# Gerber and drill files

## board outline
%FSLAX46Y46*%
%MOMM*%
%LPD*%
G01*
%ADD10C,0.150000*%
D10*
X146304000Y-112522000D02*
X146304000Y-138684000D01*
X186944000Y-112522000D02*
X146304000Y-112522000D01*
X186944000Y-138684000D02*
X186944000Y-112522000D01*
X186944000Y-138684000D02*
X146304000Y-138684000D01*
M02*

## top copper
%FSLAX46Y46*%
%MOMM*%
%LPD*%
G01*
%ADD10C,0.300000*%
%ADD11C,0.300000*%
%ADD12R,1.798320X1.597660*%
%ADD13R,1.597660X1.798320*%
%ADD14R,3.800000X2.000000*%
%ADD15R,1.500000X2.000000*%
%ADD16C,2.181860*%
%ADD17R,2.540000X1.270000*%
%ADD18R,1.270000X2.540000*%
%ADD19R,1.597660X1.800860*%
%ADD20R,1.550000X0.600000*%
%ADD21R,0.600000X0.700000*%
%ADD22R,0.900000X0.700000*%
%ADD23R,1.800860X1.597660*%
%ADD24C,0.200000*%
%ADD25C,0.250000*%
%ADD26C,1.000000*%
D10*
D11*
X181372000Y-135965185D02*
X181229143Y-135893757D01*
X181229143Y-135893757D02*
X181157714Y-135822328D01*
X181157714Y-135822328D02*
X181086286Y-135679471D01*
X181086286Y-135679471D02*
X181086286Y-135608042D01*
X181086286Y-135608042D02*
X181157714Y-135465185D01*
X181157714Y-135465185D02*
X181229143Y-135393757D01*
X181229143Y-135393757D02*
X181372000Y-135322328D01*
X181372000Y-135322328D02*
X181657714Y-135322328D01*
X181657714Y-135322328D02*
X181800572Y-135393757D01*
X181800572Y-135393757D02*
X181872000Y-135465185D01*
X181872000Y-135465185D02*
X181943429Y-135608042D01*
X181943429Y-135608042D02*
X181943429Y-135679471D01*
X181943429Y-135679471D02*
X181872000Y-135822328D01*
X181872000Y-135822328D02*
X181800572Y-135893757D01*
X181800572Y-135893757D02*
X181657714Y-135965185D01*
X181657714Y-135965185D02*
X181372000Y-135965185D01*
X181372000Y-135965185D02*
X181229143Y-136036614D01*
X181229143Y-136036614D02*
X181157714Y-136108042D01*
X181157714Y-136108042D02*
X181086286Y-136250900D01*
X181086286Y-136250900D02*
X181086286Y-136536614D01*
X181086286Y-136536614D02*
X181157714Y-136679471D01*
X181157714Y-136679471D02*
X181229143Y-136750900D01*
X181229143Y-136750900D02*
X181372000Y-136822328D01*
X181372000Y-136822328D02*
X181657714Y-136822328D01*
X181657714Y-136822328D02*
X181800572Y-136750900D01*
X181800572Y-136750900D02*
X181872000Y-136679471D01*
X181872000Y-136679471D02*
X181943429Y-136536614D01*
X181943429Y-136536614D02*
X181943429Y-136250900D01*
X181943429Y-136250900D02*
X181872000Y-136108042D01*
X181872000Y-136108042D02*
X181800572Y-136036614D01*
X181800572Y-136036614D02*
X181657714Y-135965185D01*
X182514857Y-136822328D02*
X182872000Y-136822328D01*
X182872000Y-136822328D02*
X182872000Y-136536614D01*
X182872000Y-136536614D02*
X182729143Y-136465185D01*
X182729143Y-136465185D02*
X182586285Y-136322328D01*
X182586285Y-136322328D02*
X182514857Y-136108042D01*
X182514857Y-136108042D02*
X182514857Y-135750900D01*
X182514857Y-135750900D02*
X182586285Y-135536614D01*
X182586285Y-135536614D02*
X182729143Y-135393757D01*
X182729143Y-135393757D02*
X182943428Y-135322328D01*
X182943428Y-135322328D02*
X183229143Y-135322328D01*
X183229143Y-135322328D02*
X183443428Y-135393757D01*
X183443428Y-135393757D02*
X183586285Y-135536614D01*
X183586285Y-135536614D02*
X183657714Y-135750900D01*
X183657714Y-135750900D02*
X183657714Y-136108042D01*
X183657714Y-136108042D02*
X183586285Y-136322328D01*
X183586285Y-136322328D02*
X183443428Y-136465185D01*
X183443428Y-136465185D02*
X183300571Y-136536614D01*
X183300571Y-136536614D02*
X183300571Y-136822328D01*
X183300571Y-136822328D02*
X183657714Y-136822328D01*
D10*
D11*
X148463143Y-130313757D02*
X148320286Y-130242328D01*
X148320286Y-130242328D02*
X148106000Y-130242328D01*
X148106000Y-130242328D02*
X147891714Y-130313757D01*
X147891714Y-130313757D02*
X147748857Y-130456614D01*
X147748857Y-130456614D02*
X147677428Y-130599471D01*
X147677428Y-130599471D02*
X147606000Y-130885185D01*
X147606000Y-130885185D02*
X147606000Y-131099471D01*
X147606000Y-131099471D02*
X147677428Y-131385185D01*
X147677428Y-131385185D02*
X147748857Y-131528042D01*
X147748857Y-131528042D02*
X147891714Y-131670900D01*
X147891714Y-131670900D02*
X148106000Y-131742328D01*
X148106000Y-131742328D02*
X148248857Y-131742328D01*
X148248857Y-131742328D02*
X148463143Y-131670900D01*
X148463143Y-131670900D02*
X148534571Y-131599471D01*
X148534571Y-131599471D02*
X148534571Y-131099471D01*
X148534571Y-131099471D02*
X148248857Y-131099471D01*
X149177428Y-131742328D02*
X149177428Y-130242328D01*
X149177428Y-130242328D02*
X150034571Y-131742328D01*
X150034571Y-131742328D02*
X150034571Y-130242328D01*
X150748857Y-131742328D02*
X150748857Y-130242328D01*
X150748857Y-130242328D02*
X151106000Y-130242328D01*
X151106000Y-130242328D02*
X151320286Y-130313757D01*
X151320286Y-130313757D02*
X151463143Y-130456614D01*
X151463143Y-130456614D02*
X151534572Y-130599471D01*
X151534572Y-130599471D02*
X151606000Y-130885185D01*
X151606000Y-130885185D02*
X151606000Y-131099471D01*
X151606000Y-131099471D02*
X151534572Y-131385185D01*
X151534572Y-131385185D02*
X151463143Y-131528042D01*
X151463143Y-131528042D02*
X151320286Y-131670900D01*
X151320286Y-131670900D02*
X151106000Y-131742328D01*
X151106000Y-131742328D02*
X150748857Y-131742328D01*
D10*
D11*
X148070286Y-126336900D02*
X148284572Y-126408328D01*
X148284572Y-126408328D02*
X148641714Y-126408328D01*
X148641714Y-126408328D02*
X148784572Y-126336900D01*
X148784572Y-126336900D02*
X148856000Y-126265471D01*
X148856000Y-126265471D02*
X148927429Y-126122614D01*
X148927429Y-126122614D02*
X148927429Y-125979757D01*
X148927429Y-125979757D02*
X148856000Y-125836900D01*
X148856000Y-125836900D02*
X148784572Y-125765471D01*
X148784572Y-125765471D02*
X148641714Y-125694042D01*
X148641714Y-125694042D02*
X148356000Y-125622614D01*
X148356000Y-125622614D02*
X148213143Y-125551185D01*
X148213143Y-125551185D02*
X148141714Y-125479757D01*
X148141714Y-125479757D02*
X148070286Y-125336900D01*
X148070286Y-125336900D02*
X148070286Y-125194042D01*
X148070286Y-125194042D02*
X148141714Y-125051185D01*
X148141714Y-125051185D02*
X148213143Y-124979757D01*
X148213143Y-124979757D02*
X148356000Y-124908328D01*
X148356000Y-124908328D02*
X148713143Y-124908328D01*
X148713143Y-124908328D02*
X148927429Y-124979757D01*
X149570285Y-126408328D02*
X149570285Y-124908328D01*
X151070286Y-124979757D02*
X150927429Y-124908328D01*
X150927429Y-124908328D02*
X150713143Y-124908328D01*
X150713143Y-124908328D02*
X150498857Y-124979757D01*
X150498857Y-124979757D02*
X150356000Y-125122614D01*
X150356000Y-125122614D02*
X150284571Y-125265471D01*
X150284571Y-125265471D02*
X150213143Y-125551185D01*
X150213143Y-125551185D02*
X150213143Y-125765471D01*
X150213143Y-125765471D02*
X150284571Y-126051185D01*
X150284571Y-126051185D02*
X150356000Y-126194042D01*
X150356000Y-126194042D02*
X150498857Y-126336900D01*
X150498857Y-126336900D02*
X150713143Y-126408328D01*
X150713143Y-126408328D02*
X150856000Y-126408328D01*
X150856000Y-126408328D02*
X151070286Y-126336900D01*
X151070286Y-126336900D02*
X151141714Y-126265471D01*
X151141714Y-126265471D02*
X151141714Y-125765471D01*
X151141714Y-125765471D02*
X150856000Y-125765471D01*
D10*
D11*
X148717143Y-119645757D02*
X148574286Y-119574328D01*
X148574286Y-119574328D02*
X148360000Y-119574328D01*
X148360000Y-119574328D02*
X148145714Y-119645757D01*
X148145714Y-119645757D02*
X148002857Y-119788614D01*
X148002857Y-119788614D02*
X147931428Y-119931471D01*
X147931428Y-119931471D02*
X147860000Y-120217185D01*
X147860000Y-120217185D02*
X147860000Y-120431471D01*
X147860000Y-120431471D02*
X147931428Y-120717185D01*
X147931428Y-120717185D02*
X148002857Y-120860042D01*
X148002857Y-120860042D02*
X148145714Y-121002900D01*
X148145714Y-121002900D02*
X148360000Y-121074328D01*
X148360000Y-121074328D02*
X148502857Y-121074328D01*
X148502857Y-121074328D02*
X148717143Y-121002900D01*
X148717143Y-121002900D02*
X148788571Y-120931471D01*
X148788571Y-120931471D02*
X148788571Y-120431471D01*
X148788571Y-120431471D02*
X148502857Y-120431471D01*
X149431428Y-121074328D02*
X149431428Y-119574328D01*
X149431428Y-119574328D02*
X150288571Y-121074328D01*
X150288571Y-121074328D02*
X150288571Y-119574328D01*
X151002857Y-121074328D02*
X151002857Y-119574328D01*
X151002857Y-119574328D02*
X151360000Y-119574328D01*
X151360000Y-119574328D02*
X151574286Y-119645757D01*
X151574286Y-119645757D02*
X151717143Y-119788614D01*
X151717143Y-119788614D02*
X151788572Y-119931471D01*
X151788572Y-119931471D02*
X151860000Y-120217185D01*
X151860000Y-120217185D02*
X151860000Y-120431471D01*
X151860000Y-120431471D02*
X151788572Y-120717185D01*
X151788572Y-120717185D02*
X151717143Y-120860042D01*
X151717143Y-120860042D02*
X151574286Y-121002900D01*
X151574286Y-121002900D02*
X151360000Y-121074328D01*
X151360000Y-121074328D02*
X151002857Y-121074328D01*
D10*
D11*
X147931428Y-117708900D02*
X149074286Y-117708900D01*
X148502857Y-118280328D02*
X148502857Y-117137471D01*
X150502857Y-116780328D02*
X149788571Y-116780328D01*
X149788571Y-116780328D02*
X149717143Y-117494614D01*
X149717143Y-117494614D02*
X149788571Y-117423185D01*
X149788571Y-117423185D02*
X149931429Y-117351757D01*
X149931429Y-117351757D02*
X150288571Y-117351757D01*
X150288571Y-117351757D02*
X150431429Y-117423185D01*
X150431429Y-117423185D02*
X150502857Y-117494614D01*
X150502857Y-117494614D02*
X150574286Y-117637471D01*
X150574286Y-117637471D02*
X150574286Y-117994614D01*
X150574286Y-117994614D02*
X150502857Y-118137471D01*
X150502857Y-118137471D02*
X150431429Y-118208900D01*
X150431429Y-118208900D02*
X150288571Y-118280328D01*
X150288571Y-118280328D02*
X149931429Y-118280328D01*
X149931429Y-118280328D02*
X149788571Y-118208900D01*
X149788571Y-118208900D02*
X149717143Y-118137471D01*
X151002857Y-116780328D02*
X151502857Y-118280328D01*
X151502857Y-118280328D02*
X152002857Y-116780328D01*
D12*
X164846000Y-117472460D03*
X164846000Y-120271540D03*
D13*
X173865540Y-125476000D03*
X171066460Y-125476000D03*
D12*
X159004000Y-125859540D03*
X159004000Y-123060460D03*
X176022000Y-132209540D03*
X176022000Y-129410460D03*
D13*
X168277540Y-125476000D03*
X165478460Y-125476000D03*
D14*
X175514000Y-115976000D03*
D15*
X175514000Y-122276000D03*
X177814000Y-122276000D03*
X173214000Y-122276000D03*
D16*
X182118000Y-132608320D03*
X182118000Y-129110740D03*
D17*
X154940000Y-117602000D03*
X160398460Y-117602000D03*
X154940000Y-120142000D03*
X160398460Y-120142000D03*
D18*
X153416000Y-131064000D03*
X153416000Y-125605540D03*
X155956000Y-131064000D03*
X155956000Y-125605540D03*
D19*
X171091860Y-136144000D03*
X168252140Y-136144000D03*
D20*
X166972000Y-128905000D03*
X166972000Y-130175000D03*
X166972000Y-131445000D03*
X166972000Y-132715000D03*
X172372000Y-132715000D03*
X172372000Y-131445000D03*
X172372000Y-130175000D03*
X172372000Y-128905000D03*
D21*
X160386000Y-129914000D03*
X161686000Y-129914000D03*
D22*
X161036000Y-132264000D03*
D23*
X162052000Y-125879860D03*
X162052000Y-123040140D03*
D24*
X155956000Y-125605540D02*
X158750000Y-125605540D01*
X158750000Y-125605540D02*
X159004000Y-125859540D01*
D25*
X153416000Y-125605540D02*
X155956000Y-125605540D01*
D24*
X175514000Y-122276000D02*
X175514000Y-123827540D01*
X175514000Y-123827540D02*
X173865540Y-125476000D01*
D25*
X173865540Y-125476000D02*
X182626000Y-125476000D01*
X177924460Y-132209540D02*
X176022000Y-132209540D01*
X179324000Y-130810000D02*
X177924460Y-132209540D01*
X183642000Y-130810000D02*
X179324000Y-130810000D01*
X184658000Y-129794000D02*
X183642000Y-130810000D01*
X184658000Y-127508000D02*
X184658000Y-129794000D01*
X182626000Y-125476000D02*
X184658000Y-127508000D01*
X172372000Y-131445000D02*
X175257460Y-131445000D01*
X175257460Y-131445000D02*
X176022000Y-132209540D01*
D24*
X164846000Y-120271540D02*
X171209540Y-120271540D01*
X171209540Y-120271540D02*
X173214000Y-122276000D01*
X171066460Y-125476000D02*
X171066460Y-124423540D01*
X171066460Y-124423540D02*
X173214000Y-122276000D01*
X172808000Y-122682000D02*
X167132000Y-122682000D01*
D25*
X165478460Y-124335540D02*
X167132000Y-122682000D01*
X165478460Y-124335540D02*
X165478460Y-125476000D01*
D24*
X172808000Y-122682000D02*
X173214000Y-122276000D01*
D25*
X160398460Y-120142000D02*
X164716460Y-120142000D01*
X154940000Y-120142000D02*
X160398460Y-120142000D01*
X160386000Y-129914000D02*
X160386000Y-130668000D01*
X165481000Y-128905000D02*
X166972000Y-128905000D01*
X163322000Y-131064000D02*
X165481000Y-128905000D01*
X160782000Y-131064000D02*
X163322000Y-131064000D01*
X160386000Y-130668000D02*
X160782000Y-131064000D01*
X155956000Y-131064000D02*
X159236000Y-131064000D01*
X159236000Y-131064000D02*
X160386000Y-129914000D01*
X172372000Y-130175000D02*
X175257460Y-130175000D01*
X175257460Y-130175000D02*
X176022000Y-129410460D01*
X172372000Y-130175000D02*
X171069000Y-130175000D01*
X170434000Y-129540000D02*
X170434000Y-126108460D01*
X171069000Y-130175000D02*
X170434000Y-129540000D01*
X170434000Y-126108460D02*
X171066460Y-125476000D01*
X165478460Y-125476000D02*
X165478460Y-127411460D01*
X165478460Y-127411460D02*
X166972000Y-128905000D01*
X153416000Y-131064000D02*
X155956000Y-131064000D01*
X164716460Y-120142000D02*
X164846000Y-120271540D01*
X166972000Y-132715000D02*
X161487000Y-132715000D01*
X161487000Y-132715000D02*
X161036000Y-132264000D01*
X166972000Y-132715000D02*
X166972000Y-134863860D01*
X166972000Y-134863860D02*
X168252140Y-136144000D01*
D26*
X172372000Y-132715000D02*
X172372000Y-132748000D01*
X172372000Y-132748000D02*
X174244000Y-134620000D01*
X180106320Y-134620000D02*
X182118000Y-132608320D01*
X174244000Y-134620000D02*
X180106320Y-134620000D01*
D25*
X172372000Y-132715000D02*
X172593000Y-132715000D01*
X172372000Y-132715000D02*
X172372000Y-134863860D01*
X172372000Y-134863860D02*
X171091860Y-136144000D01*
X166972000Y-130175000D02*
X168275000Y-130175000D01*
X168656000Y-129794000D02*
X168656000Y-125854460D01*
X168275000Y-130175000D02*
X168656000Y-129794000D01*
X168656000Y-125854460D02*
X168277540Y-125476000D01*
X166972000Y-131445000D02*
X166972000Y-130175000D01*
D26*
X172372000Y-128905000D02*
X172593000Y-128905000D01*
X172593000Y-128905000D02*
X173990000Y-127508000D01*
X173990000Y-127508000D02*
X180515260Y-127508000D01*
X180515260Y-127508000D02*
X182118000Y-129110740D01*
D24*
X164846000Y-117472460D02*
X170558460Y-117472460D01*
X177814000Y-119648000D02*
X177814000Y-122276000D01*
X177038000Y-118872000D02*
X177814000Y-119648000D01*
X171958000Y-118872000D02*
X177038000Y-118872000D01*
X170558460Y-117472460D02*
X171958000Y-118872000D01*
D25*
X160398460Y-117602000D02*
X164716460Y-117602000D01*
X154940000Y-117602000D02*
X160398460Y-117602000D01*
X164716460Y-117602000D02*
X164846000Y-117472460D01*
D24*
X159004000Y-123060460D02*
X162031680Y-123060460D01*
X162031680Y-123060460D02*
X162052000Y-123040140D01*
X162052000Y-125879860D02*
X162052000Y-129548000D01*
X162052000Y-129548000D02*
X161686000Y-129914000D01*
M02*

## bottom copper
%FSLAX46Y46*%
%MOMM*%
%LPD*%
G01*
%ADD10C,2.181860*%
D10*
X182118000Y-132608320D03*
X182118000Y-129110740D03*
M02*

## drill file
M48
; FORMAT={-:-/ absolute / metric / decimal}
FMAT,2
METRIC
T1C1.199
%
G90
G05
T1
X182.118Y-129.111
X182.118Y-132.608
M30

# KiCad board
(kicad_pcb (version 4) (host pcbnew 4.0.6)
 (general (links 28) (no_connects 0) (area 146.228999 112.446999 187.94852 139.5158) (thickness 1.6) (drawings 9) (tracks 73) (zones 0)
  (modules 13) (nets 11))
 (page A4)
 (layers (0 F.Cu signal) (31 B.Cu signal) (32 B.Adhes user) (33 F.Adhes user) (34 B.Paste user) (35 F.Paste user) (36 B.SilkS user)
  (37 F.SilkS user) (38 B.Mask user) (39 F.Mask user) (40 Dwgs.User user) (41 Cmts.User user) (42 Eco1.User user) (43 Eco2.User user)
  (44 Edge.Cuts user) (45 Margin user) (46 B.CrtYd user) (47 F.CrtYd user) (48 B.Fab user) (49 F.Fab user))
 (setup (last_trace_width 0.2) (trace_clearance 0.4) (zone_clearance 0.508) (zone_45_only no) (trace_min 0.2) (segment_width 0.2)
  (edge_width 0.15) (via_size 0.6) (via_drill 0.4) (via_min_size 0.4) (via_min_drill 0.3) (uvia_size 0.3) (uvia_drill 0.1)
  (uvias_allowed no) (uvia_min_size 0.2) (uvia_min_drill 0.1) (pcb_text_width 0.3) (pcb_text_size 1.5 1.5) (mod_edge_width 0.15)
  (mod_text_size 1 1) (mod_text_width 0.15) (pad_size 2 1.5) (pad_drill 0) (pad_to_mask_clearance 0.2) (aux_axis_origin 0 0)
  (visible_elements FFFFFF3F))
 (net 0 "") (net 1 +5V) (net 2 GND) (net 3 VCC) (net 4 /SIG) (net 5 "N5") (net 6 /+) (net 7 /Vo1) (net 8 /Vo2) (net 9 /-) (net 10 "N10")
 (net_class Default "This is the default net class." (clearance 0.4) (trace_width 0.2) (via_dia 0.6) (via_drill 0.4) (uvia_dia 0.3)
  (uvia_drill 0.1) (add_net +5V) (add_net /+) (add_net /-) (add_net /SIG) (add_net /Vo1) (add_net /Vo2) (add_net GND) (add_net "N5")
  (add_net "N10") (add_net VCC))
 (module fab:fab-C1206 (layer F.Cu) (at 164.846 118.872 270)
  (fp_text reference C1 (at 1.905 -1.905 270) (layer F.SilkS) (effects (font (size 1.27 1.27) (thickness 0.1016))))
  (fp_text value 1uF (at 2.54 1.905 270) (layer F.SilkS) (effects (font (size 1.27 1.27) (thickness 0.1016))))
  (pad 1 smd rect (at -1.39954 0 270) (size 1.59766 1.79832) (layers F.Cu F.Paste F.Mask) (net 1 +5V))
  (pad 2 smd rect (at 1.39954 0 270) (size 1.59766 1.79832) (layers F.Cu F.Paste F.Mask) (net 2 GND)))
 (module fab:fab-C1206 (layer F.Cu) (at 172.466 125.476 180)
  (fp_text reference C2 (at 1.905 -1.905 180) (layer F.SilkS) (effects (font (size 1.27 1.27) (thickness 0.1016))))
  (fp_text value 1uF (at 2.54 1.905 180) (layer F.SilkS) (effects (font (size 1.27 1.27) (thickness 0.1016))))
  (pad 1 smd rect (at -1.39954 0 180) (size 1.59766 1.79832) (layers F.Cu F.Paste F.Mask) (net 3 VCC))
  (pad 2 smd rect (at 1.39954 0 180) (size 1.59766 1.79832) (layers F.Cu F.Paste F.Mask) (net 2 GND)))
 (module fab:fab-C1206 (layer F.Cu) (at 159.004 124.46 90)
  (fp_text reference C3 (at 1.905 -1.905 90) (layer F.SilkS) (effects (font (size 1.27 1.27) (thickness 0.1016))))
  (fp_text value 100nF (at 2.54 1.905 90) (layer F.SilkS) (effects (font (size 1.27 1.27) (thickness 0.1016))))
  (pad 1 smd rect (at -1.39954 0 90) (size 1.59766 1.79832) (layers F.Cu F.Paste F.Mask) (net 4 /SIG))
  (pad 2 smd rect (at 1.39954 0 90) (size 1.59766 1.79832) (layers F.Cu F.Paste F.Mask) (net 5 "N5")))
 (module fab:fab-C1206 (layer F.Cu) (at 176.022 130.81 90)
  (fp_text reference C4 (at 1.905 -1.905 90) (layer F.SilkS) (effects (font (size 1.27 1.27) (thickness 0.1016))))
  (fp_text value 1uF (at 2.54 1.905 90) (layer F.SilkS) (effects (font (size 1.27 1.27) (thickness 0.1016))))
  (pad 1 smd rect (at -1.39954 0 90) (size 1.59766 1.79832) (layers F.Cu F.Paste F.Mask) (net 3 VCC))
  (pad 2 smd rect (at 1.39954 0 90) (size 1.59766 1.79832) (layers F.Cu F.Paste F.Mask) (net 2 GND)))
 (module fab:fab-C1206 (layer F.Cu) (at 166.878 125.476 180)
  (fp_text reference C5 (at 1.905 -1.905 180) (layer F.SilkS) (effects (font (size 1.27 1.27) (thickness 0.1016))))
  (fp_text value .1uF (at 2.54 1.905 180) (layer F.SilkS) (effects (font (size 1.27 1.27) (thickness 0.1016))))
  (pad 1 smd rect (at -1.39954 0 180) (size 1.59766 1.79832) (layers F.Cu F.Paste F.Mask) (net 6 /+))
  (pad 2 smd rect (at 1.39954 0 180) (size 1.59766 1.79832) (layers F.Cu F.Paste F.Mask) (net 2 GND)))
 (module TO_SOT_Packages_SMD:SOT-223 (layer F.Cu) (at 175.514 119.126 90)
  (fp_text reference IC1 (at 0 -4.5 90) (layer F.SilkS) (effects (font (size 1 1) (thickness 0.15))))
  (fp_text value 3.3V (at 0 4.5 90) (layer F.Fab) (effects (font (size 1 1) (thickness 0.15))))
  (pad 4 smd rect (at 3.15 0 90) (size 2 3.8) (layers F.Cu F.Paste F.Mask))
  (pad 1 smd rect (at -3.15 0 90) (size 2 1.5) (layers F.Cu F.Paste F.Mask) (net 3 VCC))
  (pad 2 smd rect (at -3.15 2.3 90) (size 2 1.5) (layers F.Cu F.Paste F.Mask) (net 1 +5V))
  (pad 3 smd rect (at -3.15 -2.3 90) (size 2 1.5) (layers F.Cu F.Paste F.Mask) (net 2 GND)))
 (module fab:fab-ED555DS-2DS (layer F.Cu) (at 182.118 130.81 270)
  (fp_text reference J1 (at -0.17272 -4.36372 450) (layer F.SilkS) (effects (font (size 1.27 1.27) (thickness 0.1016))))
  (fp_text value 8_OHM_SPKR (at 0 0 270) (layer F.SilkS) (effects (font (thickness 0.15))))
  (pad 1 thru_hole circle (at 1.79832 0 270) (size 2.18186 2.18186) (drill 1.19888) (layers *.Cu F.Paste F.SilkS F.Mask) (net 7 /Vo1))
  (pad 2 thru_hole circle (at -1.69926 0 270) (size 2.18186 2.18186) (drill 1.19888) (layers *.Cu F.Paste F.SilkS F.Mask) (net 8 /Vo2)))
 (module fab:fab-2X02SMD (layer F.Cu) (at 157.48 118.872)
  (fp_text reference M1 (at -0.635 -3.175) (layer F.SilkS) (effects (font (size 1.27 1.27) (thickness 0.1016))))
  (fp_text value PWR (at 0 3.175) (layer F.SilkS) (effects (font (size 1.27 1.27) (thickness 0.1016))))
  (pad 1 smd rect (at -2.54 -1.27) (size 2.54 1.27) (layers F.Cu F.Paste F.Mask) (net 1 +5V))
  (pad 2 smd rect (at 2.91846 -1.27) (size 2.54 1.27) (layers F.Cu F.Paste F.Mask) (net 1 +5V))
  (pad 3 smd rect (at -2.54 1.27) (size 2.54 1.27) (layers F.Cu F.Paste F.Mask) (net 2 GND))
  (pad 4 smd rect (at 2.91846 1.27) (size 2.54 1.27) (layers F.Cu F.Paste F.Mask) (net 2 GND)))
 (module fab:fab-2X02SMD (layer F.Cu) (at 154.686 128.524 90)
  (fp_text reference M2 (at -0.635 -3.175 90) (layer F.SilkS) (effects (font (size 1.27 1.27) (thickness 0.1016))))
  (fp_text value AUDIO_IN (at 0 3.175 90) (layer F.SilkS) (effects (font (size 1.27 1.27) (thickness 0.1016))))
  (pad 1 smd rect (at -2.54 -1.27 90) (size 2.54 1.27) (layers F.Cu F.Paste F.Mask) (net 2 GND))
  (pad 2 smd rect (at 2.91846 -1.27 90) (size 2.54 1.27) (layers F.Cu F.Paste F.Mask) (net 4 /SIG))
  (pad 3 smd rect (at -2.54 1.27 90) (size 2.54 1.27) (layers F.Cu F.Paste F.Mask) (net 2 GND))
  (pad 4 smd rect (at 2.91846 1.27 90) (size 2.54 1.27) (layers F.Cu F.Paste F.Mask) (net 4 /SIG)))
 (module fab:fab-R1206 (layer F.Cu) (at 169.672 136.144 180)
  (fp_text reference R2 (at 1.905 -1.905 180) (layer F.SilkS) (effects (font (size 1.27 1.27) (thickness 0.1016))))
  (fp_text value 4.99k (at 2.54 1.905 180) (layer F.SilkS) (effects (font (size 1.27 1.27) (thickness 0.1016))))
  (pad 1 smd rect (at -1.41986 0 180) (size 1.59766 1.80086) (layers F.Cu F.Paste F.Mask) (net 7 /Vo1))
  (pad 2 smd rect (at 1.41986 0 180) (size 1.59766 1.80086) (layers F.Cu F.Paste F.Mask) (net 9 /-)))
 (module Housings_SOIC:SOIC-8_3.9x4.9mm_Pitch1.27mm (layer F.Cu) (at 169.672 130.81)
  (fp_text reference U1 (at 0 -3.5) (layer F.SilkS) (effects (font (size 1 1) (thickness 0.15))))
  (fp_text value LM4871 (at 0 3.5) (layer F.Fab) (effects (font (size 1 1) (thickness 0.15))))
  (pad 1 smd rect (at -2.7 -1.905) (size 1.55 0.6) (layers F.Cu F.Paste F.Mask) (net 2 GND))
  (pad 2 smd rect (at -2.7 -0.635) (size 1.55 0.6) (layers F.Cu F.Paste F.Mask) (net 6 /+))
  (pad 3 smd rect (at -2.7 0.635) (size 1.55 0.6) (layers F.Cu F.Paste F.Mask) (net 6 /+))
  (pad 4 smd rect (at -2.7 1.905) (size 1.55 0.6) (layers F.Cu F.Paste F.Mask) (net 9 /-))
  (pad 5 smd rect (at 2.7 1.905) (size 1.55 0.6) (layers F.Cu F.Paste F.Mask) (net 7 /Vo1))
  (pad 6 smd rect (at 2.7 0.635) (size 1.55 0.6) (layers F.Cu F.Paste F.Mask) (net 3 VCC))
  (pad 7 smd rect (at 2.7 -0.635) (size 1.55 0.6) (layers F.Cu F.Paste F.Mask) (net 2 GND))
  (pad 8 smd rect (at 2.7 -1.905) (size 1.55 0.6) (layers F.Cu F.Paste F.Mask) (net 8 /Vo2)))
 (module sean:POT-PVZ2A (layer F.Cu) (at 161.036 131.064 180)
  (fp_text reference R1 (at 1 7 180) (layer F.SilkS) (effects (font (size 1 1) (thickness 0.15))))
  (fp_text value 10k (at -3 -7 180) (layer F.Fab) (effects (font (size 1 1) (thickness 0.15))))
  (pad 3 smd rect (at 0.65 1.15 180) (size 0.6 0.7) (layers F.Cu F.Paste F.Mask) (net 2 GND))
  (pad 1 smd rect (at -0.65 1.15 180) (size 0.6 0.7) (layers F.Cu F.Paste F.Mask) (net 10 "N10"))
  (pad 2 smd rect (at 0 -1.2 180) (size 0.9 0.7) (layers F.Cu F.Paste F.Mask) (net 9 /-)))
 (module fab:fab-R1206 (layer F.Cu) (at 162.052 124.46 90)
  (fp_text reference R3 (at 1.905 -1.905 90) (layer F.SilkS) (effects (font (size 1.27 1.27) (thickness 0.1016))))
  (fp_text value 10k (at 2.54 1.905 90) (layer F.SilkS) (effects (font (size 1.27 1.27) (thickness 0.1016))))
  (pad 1 smd rect (at -1.41986 0 90) (size 1.59766 1.80086) (layers F.Cu F.Paste F.Mask) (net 10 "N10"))
  (pad 2 smd rect (at 1.41986 0 90) (size 1.59766 1.80086) (layers F.Cu F.Paste F.Mask) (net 5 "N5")))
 (gr_line (start 146.304 112.522) (end 146.304 138.684) (angle 90) (layer Edge.Cuts) (width 0.15))
 (gr_line (start 186.944 112.522) (end 146.304 112.522) (angle 90) (layer Edge.Cuts) (width 0.15))
 (gr_line (start 186.944 138.684) (end 186.944 112.522) (angle 90) (layer Edge.Cuts) (width 0.15))
 (gr_line (start 186.944 138.684) (end 146.304 138.684) (angle 90) (layer Edge.Cuts) (width 0.15))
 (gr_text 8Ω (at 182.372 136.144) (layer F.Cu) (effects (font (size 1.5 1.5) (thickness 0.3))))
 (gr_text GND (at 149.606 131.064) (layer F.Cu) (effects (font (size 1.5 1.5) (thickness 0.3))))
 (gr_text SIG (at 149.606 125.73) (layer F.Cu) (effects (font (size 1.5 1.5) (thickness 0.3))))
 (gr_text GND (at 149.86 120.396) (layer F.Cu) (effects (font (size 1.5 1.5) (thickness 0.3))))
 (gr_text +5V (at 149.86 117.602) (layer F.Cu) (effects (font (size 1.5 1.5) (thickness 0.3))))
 (segment (start 155.956 125.60554) (end 158.75 125.60554) (width 0.2) (layer F.Cu) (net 4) (status C00000))
 (segment (start 158.75 125.60554) (end 159.004 125.85954) (width 0.2) (layer F.Cu) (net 4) (status C00000))
 (segment (start 153.416 125.60554) (end 155.956 125.60554) (width 0.25) (layer F.Cu) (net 4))
 (segment (start 175.514 122.276) (end 175.514 123.82754) (width 0.2) (layer F.Cu) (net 3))
 (segment (start 175.514 123.82754) (end 173.86554 125.476) (width 0.2) (layer F.Cu) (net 3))
 (segment (start 173.86554 125.476) (end 182.626 125.476) (width 0.25) (layer F.Cu) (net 3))
 (segment (start 177.92446 132.20954) (end 176.022 132.20954) (width 0.25) (layer F.Cu) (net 3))
 (segment (start 179.324 130.81) (end 177.92446 132.20954) (width 0.25) (layer F.Cu) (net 3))
 (segment (start 183.642 130.81) (end 179.324 130.81) (width 0.25) (layer F.Cu) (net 3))
 (segment (start 184.658 129.794) (end 183.642 130.81) (width 0.25) (layer F.Cu) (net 3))
 (segment (start 184.658 127.508) (end 184.658 129.794) (width 0.25) (layer F.Cu) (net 3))
 (segment (start 182.626 125.476) (end 184.658 127.508) (width 0.25) (layer F.Cu) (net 3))
 (segment (start 172.372 131.445) (end 175.25746 131.445) (width 0.25) (layer F.Cu) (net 3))
 (segment (start 175.25746 131.445) (end 176.022 132.20954) (width 0.25) (layer F.Cu) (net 3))
 (segment (start 164.846 120.27154) (end 171.20954 120.27154) (width 0.2) (layer F.Cu) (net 2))
 (segment (start 171.20954 120.27154) (end 173.214 122.276) (width 0.2) (layer F.Cu) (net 2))
 (segment (start 171.06646 125.476) (end 171.06646 124.42354) (width 0.2) (layer F.Cu) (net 2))
 (segment (start 171.06646 124.42354) (end 173.214 122.276) (width 0.2) (layer F.Cu) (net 2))
 (segment (start 172.808 122.682) (end 167.132 122.682) (width 0.2) (layer F.Cu) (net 2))
 (segment (start 165.47846 124.33554) (end 167.132 122.682) (width 0.25) (layer F.Cu) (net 2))
 (segment (start 165.47846 124.33554) (end 165.47846 125.476) (width 0.25) (layer F.Cu) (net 2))
 (segment (start 172.808 122.682) (end 173.214 122.276) (width 0.2) (layer F.Cu) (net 2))
 (segment (start 160.39846 120.142) (end 164.71646 120.142) (width 0.25) (layer F.Cu) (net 2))
 (segment (start 154.94 120.142) (end 160.39846 120.142) (width 0.25) (layer F.Cu) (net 2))
 (segment (start 160.386 129.914) (end 160.386 130.668) (width 0.25) (layer F.Cu) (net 2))
 (segment (start 165.481 128.905) (end 166.972 128.905) (width 0.25) (layer F.Cu) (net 2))
 (segment (start 163.322 131.064) (end 165.481 128.905) (width 0.25) (layer F.Cu) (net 2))
 (segment (start 160.782 131.064) (end 163.322 131.064) (width 0.25) (layer F.Cu) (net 2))
 (segment (start 160.386 130.668) (end 160.782 131.064) (width 0.25) (layer F.Cu) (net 2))
 (segment (start 155.956 131.064) (end 159.236 131.064) (width 0.25) (layer F.Cu) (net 2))
 (segment (start 159.236 131.064) (end 160.386 129.914) (width 0.25) (layer F.Cu) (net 2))
 (segment (start 172.372 130.175) (end 175.25746 130.175) (width 0.25) (layer F.Cu) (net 2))
 (segment (start 175.25746 130.175) (end 176.022 129.41046) (width 0.25) (layer F.Cu) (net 2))
 (segment (start 172.372 130.175) (end 171.069 130.175) (width 0.25) (layer F.Cu) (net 2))
 (segment (start 170.434 129.54) (end 170.434 126.10846) (width 0.25) (layer F.Cu) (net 2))
 (segment (start 171.069 130.175) (end 170.434 129.54) (width 0.25) (layer F.Cu) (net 2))
 (segment (start 170.434 126.10846) (end 171.06646 125.476) (width 0.25) (layer F.Cu) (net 2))
 (segment (start 165.47846 125.476) (end 165.47846 127.41146) (width 0.25) (layer F.Cu) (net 2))
 (segment (start 165.47846 127.41146) (end 166.972 128.905) (width 0.25) (layer F.Cu) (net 2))
 (segment (start 153.416 131.064) (end 155.956 131.064) (width 0.25) (layer F.Cu) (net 2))
 (segment (start 164.71646 120.142) (end 164.846 120.27154) (width 0.25) (layer F.Cu) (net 2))
 (segment (start 166.972 132.715) (end 161.487 132.715) (width 0.25) (layer F.Cu) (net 9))
 (segment (start 161.487 132.715) (end 161.036 132.264) (width 0.25) (layer F.Cu) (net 9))
 (segment (start 166.972 132.715) (end 166.972 134.86386) (width 0.25) (layer F.Cu) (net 9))
 (segment (start 166.972 134.86386) (end 168.25214 136.144) (width 0.25) (layer F.Cu) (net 9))
 (segment (start 172.372 132.715) (end 172.372 132.748) (width 1) (layer F.Cu) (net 7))
 (segment (start 172.372 132.748) (end 174.244 134.62) (width 1) (layer F.Cu) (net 7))
 (segment (start 180.10632 134.62) (end 182.118 132.60832) (width 1) (layer F.Cu) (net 7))
 (segment (start 174.244 134.62) (end 180.10632 134.62) (width 1) (layer F.Cu) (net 7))
 (segment (start 172.372 132.715) (end 172.593 132.715) (width 0.25) (layer F.Cu) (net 7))
 (segment (start 172.372 132.715) (end 172.372 134.86386) (width 0.25) (layer F.Cu) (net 7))
 (segment (start 172.372 134.86386) (end 171.09186 136.144) (width 0.25) (layer F.Cu) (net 7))
 (segment (start 166.972 130.175) (end 168.275 130.175) (width 0.25) (layer F.Cu) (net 6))
 (segment (start 168.656 129.794) (end 168.656 125.85446) (width 0.25) (layer F.Cu) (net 6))
 (segment (start 168.275 130.175) (end 168.656 129.794) (width 0.25) (layer F.Cu) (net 6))
 (segment (start 168.656 125.85446) (end 168.27754 125.476) (width 0.25) (layer F.Cu) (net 6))
 (segment (start 166.972 131.445) (end 166.972 130.175) (width 0.25) (layer F.Cu) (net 6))
 (segment (start 172.372 128.905) (end 172.593 128.905) (width 1) (layer F.Cu) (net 8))
 (segment (start 172.593 128.905) (end 173.99 127.508) (width 1) (layer F.Cu) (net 8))
 (segment (start 173.99 127.508) (end 180.51526 127.508) (width 1) (layer F.Cu) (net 8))
 (segment (start 180.51526 127.508) (end 182.118 129.11074) (width 1) (layer F.Cu) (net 8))
 (segment (start 164.846 117.47246) (end 170.55846 117.47246) (width 0.2) (layer F.Cu) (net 1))
 (segment (start 177.814 119.648) (end 177.814 122.276) (width 0.2) (layer F.Cu) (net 1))
 (segment (start 177.038 118.872) (end 177.814 119.648) (width 0.2) (layer F.Cu) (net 1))
 (segment (start 171.958 118.872) (end 177.038 118.872) (width 0.2) (layer F.Cu) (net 1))
 (segment (start 170.55846 117.47246) (end 171.958 118.872) (width 0.2) (layer F.Cu) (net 1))
 (segment (start 160.39846 117.602) (end 164.71646 117.602) (width 0.25) (layer F.Cu) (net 1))
 (segment (start 154.94 117.602) (end 160.39846 117.602) (width 0.25) (layer F.Cu) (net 1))
 (segment (start 164.71646 117.602) (end 164.846 117.47246) (width 0.25) (layer F.Cu) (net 1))
 (segment (start 159.004 123.06046) (end 162.03168 123.06046) (width 0.2) (layer F.Cu) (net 5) (status C00000))
 (segment (start 162.03168 123.06046) (end 162.052 123.04014) (width 0.2) (layer F.Cu) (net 5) (status C00000))
 (segment (start 162.052 125.87986) (end 162.052 129.548) (width 0.2) (layer F.Cu) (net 10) (status 400000))
 (segment (start 162.052 129.548) (end 161.686 129.914) (width 0.2) (layer F.Cu) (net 10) (status 800000)))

